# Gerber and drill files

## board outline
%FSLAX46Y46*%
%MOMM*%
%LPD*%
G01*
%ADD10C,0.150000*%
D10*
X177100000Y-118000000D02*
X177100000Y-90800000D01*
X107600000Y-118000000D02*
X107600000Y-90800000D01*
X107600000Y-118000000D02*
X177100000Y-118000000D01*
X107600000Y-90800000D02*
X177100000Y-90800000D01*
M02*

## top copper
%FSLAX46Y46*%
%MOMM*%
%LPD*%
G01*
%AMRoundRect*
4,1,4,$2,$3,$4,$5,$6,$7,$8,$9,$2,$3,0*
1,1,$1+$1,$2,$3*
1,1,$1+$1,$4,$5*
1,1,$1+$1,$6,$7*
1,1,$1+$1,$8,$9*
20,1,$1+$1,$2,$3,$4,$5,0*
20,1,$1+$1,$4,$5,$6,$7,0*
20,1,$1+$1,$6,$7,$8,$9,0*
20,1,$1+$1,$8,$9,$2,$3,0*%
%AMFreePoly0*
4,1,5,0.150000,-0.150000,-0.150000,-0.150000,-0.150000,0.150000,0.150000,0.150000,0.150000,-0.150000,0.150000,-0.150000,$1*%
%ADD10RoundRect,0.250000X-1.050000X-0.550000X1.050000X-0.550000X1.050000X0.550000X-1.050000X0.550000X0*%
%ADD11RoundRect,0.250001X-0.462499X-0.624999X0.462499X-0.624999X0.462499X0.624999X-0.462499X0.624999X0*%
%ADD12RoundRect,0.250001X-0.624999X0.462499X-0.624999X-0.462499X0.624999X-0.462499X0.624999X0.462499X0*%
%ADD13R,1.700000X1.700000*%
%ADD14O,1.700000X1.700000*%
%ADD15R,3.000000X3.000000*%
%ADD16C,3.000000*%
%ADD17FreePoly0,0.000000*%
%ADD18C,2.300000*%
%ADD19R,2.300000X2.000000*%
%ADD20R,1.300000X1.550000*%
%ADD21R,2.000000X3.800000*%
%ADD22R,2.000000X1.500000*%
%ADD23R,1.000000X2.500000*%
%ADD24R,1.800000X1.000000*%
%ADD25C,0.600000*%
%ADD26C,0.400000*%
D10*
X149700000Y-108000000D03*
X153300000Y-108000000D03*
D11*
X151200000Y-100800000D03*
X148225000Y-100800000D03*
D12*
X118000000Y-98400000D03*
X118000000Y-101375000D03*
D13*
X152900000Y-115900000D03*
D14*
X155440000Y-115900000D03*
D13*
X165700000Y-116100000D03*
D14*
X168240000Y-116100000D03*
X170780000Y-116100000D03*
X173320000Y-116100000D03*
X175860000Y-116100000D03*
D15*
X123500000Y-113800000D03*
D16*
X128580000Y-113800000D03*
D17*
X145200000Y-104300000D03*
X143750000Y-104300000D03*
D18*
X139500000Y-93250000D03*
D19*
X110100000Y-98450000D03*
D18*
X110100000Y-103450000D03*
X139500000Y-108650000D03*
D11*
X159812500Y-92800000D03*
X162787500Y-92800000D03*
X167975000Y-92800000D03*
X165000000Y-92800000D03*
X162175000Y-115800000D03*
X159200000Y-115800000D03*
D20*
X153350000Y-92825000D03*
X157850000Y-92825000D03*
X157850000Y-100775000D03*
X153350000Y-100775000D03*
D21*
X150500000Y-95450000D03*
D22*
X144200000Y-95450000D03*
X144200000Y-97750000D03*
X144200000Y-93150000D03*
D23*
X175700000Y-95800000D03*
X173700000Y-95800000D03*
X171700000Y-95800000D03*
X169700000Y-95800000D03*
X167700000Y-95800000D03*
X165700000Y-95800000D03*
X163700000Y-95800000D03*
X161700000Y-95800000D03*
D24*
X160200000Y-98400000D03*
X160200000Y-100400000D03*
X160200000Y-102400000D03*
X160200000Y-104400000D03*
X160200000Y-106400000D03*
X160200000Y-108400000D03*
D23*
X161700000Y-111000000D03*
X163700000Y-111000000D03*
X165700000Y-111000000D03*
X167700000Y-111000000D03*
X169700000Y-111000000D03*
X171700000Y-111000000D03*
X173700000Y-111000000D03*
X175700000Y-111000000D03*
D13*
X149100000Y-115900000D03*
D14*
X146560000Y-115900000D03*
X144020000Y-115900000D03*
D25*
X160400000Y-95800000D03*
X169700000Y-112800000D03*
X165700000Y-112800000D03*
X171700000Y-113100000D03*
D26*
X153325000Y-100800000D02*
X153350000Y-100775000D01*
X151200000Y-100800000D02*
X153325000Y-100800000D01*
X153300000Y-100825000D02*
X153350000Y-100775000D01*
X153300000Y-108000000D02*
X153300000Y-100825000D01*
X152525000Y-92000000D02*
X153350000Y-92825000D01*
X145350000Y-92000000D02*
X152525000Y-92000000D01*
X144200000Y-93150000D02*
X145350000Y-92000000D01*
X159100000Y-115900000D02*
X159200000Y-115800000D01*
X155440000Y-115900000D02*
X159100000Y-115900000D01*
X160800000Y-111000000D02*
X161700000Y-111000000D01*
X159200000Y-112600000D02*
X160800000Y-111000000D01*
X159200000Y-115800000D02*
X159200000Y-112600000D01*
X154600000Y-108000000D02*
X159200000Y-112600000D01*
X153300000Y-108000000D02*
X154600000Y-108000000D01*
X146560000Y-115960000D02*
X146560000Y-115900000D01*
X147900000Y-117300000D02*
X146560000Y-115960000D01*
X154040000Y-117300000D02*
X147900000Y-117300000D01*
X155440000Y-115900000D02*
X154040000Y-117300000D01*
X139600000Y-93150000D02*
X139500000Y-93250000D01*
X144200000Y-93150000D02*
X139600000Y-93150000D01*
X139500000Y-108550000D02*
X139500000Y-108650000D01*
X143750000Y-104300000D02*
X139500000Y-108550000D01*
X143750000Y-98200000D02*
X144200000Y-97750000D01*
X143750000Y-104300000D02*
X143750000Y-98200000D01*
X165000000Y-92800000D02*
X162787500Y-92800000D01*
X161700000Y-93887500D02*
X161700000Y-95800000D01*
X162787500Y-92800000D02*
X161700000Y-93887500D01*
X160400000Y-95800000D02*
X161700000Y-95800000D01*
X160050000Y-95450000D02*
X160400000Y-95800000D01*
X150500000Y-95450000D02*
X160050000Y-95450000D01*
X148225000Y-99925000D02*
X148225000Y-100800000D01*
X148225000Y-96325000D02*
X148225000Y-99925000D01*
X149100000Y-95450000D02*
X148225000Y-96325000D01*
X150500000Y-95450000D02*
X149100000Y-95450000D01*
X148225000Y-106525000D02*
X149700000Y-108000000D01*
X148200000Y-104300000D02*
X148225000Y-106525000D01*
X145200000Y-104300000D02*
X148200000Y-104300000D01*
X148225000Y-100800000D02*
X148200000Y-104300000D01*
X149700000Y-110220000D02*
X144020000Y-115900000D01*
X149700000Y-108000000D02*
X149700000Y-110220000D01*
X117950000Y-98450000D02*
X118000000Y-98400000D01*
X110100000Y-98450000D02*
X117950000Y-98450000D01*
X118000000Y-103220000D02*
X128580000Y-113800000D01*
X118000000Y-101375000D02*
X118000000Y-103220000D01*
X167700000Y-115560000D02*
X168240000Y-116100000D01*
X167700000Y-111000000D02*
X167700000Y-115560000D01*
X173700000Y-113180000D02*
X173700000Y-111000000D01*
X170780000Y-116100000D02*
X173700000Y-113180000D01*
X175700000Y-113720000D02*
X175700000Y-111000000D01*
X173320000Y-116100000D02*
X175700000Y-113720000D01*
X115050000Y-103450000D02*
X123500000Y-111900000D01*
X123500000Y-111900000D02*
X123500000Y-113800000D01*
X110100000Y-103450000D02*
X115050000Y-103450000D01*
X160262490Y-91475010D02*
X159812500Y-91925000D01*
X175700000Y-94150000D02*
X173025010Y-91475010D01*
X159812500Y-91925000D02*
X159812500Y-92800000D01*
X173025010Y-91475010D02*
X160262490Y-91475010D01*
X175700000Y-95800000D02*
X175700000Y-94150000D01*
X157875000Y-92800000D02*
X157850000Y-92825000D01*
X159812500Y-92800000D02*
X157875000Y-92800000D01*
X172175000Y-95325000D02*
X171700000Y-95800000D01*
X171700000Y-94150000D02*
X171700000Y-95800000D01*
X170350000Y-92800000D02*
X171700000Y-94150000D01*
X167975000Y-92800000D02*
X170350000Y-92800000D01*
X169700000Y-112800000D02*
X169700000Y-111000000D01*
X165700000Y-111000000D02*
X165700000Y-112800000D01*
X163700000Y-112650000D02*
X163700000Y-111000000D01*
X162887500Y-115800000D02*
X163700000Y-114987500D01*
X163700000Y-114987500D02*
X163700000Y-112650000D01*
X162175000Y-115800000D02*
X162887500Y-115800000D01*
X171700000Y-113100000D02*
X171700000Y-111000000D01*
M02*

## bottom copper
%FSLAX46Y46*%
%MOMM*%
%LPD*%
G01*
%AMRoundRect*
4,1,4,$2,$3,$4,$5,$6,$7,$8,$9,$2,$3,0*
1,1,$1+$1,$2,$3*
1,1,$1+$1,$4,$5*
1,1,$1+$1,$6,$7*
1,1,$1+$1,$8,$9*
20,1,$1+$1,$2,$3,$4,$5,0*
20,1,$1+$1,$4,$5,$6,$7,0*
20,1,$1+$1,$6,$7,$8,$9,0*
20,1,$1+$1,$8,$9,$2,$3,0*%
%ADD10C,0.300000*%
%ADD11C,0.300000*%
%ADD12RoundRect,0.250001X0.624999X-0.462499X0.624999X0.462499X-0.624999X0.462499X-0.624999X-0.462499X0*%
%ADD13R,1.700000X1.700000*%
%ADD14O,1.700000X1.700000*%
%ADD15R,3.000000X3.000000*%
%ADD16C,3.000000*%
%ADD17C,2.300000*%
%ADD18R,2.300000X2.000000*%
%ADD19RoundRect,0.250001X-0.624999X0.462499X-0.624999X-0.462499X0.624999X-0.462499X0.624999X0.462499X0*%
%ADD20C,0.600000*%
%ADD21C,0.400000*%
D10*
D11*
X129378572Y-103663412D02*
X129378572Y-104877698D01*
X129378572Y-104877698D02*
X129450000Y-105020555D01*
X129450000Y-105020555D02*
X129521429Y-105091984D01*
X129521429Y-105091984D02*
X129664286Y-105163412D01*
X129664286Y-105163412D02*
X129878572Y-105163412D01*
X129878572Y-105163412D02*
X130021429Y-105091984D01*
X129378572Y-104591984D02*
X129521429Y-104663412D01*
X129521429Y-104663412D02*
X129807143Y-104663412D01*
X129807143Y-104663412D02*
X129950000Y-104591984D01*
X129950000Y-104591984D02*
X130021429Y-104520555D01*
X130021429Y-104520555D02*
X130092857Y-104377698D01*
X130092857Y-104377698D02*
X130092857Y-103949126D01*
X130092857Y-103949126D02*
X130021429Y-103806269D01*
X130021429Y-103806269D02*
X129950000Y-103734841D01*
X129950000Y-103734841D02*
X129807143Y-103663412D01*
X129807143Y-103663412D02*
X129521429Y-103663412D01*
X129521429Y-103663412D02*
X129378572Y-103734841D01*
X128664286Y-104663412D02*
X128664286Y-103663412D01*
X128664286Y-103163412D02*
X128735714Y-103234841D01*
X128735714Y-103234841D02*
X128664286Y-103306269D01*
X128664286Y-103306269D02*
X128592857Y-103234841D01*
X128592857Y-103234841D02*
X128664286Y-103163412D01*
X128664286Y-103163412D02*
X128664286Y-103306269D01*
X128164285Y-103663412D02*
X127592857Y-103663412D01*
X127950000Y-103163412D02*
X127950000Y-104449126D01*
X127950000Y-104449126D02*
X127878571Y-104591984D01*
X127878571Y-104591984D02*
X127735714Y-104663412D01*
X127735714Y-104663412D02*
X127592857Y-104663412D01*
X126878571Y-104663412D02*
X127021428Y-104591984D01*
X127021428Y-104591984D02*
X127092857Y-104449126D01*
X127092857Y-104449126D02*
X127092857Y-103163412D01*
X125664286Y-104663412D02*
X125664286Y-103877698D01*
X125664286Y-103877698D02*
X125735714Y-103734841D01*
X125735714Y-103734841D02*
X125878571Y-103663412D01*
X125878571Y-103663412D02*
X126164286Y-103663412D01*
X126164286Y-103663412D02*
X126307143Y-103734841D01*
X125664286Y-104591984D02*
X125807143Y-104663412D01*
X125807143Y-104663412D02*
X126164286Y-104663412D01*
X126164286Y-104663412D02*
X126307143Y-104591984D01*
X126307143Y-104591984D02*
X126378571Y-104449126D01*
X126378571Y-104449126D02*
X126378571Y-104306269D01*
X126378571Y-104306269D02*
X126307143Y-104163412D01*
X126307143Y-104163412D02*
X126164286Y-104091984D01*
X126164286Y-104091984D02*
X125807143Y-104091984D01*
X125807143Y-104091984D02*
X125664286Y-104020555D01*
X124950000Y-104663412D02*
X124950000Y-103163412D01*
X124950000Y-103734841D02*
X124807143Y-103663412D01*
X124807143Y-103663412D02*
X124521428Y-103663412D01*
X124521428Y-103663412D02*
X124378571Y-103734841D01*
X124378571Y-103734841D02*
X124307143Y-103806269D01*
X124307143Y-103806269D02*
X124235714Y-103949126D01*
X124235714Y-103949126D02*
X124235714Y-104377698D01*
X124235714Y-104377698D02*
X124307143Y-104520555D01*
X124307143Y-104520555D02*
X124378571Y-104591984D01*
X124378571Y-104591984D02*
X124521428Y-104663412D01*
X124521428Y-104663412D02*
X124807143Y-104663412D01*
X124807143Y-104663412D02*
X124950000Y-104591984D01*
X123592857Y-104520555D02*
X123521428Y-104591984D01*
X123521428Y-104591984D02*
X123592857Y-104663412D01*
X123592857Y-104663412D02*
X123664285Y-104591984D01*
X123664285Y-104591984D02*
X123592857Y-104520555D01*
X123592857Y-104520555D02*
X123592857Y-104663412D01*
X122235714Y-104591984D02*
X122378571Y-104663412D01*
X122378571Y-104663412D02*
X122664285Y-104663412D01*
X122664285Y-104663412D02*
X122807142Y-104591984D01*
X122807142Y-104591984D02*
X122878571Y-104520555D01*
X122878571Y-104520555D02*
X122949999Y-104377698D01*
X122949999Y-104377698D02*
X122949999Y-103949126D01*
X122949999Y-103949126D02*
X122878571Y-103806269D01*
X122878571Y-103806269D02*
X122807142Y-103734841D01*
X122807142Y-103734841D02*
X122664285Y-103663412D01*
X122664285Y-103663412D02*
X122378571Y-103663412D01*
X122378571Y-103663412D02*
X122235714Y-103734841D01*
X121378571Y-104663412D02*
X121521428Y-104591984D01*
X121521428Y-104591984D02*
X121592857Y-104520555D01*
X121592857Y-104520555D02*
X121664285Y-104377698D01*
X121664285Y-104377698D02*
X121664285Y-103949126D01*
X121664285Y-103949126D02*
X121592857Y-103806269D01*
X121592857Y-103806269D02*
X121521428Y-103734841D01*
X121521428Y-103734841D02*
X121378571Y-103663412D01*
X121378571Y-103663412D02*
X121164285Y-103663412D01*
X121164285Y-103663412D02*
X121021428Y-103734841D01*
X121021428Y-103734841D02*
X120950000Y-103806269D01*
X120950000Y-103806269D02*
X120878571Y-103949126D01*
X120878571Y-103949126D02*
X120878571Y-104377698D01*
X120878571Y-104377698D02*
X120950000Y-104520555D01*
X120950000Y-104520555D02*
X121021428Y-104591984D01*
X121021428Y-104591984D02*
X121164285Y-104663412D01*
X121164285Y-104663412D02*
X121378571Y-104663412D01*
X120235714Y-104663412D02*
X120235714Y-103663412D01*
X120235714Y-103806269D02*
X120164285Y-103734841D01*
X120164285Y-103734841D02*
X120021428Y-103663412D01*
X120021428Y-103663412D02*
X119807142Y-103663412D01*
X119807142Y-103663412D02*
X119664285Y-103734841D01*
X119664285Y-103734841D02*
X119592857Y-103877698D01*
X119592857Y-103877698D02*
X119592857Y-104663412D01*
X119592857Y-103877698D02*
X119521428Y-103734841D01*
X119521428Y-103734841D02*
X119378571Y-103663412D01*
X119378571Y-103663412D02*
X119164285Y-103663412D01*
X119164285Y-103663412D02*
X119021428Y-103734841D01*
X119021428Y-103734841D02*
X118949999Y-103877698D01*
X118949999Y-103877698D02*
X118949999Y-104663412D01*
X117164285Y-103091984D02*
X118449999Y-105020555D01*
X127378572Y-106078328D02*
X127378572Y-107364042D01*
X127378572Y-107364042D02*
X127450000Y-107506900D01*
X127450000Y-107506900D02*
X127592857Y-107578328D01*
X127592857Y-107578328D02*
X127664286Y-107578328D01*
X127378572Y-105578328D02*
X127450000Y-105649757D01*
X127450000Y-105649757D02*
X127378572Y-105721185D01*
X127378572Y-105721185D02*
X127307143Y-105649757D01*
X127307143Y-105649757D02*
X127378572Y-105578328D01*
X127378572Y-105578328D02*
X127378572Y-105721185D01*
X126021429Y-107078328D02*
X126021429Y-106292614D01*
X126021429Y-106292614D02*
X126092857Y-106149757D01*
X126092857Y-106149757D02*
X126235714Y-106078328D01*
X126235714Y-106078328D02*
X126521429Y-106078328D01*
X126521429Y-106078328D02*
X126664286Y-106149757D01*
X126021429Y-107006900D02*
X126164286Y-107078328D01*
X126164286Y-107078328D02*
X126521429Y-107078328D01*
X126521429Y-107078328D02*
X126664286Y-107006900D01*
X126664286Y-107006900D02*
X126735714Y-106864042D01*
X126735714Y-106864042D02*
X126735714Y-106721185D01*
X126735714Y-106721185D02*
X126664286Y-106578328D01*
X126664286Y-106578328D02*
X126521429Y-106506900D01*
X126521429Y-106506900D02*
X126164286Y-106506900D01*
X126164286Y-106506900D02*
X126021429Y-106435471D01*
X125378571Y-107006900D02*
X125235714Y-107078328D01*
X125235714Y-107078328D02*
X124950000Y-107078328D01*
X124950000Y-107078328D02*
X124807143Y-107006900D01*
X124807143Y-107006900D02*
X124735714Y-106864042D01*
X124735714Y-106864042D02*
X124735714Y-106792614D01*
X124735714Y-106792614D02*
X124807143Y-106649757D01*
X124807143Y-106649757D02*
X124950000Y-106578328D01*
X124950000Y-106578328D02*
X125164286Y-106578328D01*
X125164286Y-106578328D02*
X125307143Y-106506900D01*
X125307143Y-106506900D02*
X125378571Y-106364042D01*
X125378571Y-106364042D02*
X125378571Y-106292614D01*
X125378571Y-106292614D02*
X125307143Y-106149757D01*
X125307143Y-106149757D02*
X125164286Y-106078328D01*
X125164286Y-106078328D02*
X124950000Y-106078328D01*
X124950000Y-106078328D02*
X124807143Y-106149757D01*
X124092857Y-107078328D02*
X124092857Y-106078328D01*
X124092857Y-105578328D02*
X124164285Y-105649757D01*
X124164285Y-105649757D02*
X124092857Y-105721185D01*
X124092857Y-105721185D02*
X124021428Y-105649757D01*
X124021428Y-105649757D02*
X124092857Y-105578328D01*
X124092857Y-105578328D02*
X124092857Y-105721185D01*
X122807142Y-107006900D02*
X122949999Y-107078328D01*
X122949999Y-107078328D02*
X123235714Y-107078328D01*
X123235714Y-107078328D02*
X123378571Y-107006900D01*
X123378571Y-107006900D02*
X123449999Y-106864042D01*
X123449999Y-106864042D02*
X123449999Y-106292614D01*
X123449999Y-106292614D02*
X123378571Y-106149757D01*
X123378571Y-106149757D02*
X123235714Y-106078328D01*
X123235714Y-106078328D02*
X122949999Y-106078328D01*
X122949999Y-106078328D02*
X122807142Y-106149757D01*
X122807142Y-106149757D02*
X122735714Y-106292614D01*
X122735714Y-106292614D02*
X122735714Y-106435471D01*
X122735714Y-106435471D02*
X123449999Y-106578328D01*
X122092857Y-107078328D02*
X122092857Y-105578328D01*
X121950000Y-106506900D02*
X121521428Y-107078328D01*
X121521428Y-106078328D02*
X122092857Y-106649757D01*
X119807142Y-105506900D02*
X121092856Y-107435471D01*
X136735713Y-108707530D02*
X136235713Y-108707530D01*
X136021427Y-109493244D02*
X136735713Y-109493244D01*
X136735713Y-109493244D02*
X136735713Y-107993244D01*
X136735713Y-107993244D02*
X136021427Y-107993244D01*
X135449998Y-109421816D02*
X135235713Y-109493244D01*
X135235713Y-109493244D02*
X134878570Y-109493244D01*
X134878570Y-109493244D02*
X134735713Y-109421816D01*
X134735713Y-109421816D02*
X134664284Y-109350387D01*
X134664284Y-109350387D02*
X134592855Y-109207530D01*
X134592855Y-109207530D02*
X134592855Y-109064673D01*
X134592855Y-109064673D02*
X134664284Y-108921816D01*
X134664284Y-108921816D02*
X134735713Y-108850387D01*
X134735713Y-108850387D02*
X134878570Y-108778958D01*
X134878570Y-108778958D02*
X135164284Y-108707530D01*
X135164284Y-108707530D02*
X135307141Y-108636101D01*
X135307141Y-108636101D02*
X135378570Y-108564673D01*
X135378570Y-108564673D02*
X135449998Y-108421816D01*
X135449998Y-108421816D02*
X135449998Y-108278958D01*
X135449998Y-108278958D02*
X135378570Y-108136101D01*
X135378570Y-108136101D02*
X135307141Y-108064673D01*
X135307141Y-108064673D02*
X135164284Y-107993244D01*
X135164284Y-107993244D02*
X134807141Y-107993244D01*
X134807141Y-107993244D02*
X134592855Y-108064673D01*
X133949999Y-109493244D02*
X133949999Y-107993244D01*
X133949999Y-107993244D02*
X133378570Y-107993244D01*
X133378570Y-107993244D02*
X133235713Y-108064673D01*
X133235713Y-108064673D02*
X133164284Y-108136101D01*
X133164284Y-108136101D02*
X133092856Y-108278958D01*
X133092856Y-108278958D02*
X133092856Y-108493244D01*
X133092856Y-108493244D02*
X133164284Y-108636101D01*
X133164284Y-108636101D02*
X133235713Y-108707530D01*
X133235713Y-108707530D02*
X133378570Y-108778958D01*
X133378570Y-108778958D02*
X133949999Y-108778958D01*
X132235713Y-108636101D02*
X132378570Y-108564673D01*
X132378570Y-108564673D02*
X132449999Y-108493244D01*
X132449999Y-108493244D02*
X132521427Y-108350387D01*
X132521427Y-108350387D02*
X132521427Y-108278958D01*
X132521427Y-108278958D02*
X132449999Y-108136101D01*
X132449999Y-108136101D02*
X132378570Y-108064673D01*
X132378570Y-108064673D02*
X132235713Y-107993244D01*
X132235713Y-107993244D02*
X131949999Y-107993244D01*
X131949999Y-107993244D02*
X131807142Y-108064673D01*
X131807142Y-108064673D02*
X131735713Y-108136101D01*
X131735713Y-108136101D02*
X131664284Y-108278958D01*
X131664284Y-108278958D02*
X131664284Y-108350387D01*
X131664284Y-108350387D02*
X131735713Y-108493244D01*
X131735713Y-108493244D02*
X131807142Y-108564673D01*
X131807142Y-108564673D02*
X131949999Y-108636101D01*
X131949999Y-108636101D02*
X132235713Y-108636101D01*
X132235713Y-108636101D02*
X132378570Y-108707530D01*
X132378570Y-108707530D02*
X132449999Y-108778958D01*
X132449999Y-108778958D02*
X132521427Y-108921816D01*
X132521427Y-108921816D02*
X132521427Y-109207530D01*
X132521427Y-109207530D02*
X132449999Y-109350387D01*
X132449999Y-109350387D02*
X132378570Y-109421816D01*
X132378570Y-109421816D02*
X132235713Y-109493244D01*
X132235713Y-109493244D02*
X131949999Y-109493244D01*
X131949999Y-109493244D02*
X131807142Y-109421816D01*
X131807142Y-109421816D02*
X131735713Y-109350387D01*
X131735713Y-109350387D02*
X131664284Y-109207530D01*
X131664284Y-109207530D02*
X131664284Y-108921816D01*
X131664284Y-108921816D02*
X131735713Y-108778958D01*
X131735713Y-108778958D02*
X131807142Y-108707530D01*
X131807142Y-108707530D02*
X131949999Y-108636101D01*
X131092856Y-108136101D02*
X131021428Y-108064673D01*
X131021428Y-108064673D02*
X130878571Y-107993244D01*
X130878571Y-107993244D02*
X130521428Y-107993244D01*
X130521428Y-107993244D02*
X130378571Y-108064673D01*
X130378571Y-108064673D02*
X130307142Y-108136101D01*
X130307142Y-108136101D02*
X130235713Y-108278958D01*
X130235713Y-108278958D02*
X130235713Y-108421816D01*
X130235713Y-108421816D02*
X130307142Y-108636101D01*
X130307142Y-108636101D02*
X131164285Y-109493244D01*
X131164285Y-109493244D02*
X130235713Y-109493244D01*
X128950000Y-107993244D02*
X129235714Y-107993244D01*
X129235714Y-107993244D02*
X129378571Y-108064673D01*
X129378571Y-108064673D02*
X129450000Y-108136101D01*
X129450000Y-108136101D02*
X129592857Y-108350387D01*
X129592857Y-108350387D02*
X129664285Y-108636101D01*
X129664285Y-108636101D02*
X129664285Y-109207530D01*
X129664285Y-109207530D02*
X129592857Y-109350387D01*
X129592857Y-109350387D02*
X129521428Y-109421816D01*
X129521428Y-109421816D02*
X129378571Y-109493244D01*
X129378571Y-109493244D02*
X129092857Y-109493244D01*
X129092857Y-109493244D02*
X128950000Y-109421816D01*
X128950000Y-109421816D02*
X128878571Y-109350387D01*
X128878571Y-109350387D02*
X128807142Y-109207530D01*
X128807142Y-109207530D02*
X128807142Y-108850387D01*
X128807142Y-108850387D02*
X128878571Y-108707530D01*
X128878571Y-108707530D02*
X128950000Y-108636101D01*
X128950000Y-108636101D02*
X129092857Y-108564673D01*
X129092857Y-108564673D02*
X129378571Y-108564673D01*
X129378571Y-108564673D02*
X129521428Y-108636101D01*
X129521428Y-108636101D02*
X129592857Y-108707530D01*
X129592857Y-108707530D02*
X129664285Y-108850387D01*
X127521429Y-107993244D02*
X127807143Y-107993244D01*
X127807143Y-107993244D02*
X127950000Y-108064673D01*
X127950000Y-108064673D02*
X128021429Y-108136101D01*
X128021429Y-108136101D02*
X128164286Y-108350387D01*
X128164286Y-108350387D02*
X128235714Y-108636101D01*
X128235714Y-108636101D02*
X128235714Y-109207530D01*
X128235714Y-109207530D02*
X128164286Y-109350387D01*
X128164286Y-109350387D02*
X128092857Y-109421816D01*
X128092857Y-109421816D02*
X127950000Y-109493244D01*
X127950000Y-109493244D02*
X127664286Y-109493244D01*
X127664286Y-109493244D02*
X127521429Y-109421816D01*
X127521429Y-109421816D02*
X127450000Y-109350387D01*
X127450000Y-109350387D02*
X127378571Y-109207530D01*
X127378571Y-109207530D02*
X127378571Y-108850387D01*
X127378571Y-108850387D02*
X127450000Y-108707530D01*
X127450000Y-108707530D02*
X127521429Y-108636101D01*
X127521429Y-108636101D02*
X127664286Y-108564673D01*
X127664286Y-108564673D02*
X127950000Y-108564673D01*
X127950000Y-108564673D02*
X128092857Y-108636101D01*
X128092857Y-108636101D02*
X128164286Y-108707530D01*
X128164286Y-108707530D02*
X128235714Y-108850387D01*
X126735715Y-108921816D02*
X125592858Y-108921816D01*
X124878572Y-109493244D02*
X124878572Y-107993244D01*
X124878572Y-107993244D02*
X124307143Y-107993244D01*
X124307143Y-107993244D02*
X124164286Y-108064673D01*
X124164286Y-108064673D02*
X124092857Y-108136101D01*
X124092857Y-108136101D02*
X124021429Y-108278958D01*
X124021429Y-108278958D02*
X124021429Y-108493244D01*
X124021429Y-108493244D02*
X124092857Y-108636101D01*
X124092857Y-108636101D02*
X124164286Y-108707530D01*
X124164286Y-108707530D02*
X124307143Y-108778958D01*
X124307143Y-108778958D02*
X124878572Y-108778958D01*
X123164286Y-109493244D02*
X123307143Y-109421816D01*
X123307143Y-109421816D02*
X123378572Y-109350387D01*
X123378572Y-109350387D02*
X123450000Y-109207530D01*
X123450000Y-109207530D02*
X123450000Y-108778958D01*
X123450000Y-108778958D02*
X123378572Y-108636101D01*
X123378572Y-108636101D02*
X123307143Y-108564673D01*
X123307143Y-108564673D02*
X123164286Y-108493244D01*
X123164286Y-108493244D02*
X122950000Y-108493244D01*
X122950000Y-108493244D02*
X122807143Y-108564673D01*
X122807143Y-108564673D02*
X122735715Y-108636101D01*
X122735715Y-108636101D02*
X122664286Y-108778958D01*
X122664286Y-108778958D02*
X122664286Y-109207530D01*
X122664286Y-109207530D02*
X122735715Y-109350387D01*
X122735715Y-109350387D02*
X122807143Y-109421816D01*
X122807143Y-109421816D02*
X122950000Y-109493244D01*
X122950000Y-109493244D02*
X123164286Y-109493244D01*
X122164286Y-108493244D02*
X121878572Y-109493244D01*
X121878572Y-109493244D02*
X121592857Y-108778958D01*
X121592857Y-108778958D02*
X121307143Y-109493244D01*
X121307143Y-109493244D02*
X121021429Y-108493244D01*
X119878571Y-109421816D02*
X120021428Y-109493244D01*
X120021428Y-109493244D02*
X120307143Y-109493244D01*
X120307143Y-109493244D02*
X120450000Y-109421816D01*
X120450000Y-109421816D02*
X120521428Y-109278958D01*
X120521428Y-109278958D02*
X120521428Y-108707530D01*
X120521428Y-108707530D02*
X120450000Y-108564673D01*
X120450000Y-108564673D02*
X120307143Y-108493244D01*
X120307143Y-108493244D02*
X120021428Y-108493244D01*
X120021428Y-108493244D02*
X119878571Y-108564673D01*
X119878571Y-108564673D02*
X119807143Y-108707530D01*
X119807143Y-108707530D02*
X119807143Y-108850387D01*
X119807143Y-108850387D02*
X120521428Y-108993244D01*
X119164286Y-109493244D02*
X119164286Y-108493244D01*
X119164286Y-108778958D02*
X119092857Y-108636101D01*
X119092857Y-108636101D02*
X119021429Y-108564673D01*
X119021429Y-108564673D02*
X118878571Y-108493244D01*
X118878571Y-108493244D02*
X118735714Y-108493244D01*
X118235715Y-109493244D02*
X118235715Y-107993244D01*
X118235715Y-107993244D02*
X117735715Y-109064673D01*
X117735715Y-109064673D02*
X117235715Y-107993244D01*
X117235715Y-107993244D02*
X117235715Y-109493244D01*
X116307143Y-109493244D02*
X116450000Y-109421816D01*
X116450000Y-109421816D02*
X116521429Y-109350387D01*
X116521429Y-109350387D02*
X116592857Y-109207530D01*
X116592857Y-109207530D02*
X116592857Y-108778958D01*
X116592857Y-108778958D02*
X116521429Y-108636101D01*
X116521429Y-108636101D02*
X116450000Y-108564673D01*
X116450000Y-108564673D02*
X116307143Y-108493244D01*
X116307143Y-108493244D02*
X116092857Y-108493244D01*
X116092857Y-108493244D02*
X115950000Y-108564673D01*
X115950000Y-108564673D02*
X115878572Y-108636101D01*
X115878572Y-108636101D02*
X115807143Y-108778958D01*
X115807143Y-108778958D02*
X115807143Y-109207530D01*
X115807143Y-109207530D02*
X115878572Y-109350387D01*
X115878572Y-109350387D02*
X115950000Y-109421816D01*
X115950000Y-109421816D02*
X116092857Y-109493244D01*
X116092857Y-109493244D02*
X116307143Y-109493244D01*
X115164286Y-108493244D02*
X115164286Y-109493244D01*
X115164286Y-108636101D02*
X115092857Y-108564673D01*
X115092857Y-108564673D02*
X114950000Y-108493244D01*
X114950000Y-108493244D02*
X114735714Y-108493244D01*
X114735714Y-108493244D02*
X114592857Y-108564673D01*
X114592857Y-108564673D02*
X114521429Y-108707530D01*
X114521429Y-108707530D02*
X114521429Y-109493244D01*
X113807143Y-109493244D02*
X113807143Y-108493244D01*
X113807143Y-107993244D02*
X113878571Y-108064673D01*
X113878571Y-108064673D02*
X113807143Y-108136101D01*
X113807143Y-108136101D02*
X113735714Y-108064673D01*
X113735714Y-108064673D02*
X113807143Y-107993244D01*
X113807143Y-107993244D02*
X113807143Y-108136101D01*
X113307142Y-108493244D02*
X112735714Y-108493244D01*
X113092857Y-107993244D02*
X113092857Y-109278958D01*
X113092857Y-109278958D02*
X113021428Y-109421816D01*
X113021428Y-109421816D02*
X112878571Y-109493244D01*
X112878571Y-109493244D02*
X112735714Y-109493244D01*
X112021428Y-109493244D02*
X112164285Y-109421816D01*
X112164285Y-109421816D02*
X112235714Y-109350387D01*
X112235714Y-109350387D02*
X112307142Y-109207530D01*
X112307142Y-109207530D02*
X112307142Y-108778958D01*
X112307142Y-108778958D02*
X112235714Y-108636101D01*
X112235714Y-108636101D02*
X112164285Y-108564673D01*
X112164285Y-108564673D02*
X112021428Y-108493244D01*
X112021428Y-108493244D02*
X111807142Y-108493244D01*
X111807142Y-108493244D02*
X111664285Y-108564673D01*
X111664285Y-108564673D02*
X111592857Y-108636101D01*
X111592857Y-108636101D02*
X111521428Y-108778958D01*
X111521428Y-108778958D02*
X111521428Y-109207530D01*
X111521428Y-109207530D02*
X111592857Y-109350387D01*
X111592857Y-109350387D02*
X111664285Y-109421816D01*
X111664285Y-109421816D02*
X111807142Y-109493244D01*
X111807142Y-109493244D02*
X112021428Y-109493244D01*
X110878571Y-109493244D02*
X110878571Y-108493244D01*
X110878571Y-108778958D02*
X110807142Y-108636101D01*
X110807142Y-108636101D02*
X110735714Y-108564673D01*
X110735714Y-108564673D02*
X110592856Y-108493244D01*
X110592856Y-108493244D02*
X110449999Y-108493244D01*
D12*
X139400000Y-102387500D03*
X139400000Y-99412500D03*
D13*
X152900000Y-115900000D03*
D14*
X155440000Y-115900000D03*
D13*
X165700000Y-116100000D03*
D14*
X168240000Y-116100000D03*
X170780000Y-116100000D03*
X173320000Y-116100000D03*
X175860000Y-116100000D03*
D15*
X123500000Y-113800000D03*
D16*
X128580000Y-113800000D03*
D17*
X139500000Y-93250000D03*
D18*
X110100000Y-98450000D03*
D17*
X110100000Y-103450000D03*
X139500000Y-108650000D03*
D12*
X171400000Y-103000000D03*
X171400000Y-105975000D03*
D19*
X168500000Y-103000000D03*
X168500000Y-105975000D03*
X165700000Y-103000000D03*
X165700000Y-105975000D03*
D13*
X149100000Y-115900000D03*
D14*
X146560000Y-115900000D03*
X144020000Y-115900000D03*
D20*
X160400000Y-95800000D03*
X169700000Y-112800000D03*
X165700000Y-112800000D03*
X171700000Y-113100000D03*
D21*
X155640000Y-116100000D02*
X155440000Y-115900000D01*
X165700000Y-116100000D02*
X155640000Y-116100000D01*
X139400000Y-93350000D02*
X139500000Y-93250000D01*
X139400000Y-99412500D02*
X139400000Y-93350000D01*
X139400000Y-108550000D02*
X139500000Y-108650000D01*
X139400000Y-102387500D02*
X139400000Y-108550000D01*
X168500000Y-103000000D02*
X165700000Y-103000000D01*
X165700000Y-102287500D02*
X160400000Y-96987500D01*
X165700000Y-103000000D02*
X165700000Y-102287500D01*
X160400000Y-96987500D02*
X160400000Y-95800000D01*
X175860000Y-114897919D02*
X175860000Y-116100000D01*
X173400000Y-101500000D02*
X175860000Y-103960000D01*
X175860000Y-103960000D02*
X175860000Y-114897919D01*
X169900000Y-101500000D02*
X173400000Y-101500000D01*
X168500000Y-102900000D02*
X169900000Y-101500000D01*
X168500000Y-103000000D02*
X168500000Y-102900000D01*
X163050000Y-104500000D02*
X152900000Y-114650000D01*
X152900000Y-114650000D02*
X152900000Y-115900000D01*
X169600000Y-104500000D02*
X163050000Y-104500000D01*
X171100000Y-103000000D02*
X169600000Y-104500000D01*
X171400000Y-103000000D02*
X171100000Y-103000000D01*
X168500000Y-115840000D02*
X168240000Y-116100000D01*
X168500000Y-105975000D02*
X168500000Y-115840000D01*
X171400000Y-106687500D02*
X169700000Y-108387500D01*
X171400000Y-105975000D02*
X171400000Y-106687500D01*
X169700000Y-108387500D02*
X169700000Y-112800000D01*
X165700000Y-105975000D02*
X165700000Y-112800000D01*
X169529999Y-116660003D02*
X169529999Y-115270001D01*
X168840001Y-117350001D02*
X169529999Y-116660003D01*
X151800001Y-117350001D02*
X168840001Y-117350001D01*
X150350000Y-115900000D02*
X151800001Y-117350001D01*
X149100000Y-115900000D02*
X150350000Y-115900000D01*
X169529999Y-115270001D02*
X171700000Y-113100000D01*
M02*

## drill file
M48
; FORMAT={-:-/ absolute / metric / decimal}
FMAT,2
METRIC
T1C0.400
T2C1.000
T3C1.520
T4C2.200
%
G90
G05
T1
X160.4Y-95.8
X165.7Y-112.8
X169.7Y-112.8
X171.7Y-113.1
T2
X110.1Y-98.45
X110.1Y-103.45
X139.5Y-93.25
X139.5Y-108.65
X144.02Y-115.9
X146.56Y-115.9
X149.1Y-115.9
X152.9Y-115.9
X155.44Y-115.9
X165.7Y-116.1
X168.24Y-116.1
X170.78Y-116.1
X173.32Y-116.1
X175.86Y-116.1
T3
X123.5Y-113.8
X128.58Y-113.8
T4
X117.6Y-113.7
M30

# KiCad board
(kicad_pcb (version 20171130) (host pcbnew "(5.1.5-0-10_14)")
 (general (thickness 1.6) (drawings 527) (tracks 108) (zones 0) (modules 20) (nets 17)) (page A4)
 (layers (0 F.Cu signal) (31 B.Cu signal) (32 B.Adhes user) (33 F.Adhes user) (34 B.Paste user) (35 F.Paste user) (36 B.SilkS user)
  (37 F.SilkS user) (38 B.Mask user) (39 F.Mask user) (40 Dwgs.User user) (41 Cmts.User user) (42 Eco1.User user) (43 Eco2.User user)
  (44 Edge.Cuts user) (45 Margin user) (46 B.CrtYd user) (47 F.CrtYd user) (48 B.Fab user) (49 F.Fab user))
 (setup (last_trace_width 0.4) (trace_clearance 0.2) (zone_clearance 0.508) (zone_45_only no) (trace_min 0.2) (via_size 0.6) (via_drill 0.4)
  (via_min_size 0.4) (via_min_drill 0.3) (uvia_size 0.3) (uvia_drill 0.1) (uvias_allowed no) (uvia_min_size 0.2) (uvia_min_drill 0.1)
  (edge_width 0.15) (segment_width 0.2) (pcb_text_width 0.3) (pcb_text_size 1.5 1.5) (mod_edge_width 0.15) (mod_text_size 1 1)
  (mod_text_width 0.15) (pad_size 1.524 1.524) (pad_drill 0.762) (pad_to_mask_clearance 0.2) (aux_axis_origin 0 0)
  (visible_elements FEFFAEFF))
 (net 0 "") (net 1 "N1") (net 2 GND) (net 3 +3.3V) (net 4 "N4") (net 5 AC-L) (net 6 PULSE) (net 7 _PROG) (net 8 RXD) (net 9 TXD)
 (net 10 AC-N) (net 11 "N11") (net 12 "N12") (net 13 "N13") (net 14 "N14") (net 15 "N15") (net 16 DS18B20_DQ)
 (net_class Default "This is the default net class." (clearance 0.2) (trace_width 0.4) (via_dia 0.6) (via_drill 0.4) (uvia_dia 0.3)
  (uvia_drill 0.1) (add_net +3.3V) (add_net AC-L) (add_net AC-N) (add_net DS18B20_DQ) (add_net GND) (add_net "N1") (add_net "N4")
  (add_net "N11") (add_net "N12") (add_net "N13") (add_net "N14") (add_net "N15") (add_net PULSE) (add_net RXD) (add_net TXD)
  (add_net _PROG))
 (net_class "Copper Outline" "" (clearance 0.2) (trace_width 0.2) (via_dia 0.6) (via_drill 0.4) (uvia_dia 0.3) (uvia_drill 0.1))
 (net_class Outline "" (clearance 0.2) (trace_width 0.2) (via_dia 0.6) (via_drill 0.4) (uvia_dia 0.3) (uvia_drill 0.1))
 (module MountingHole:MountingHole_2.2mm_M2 (layer F.Cu) (at 117.6 113.7)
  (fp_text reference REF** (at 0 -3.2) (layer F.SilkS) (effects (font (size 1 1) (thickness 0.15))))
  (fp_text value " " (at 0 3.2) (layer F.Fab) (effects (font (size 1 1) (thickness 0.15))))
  (pad 1 np_thru_hole circle (at 0 0) (size 2.2 2.2) (drill 2.2) (layers *.Cu *.Mask)))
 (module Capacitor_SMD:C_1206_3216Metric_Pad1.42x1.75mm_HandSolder (layer B.Cu) (at 139.4 100.9 90)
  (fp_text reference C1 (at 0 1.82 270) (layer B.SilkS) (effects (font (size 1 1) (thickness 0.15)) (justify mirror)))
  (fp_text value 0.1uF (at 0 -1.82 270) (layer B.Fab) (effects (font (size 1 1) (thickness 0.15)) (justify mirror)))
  (pad 1 smd roundrect (at -1.4875 0 90) (size 1.425 1.75) (layers B.Cu B.Paste B.Mask) (roundrect_rratio 0.175439) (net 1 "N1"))
  (pad 2 smd roundrect (at 1.4875 0 90) (size 1.425 1.75) (layers B.Cu B.Paste B.Mask) (roundrect_rratio 0.175439) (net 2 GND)))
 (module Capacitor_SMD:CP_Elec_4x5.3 (layer F.Cu) (at 151.5 108)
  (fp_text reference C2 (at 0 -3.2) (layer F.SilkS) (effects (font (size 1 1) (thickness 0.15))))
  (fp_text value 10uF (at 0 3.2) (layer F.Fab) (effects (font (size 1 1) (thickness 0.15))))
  (pad 1 smd roundrect (at -1.8 0) (size 2.6 1.6) (layers F.Cu F.Paste F.Mask) (roundrect_rratio 0.15625) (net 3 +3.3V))
  (pad 2 smd roundrect (at 1.8 0) (size 2.6 1.6) (layers F.Cu F.Paste F.Mask) (roundrect_rratio 0.15625) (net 2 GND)))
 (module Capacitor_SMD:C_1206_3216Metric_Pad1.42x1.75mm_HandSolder (layer F.Cu) (at 149.7125 100.8)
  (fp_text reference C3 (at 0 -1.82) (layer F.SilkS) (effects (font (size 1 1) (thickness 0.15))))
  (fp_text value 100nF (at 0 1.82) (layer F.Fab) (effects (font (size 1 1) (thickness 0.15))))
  (pad 2 smd roundrect (at 1.4875 0) (size 1.425 1.75) (layers F.Cu F.Paste F.Mask) (roundrect_rratio 0.175439) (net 2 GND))
  (pad 1 smd roundrect (at -1.4875 0) (size 1.425 1.75) (layers F.Cu F.Paste F.Mask) (roundrect_rratio 0.175439) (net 3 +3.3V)))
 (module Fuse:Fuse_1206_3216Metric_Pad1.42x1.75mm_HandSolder (layer F.Cu) (at 118 99.8875 270)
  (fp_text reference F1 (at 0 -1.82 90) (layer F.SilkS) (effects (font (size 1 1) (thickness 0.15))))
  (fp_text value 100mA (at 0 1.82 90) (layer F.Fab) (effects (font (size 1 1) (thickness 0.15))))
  (pad 1 smd roundrect (at -1.4875 0 270) (size 1.425 1.75) (layers F.Cu F.Paste F.Mask) (roundrect_rratio 0.175439) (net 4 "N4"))
  (pad 2 smd roundrect (at 1.4875 0 270) (size 1.425 1.75) (layers F.Cu F.Paste F.Mask) (roundrect_rratio 0.175439) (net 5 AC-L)))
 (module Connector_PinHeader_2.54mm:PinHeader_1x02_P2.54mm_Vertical (layer F.Cu) (at 152.9 115.9 90)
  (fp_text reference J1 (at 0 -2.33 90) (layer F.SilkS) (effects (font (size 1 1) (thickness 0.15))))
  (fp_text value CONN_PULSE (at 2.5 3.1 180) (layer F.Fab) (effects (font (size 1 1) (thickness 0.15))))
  (pad 1 thru_hole rect (at 0 0 90) (size 1.7 1.7) (drill 1) (layers *.Cu *.Mask) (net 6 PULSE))
  (pad 2 thru_hole oval (at 0 2.54 90) (size 1.7 1.7) (drill 1) (layers *.Cu *.Mask) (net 2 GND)))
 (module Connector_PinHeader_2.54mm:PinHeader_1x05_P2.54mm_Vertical (layer F.Cu) (at 165.7 116.1 90)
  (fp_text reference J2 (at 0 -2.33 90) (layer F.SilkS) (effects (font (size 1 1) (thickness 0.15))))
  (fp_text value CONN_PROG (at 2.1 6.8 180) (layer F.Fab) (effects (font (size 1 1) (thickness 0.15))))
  (pad 1 thru_hole rect (at 0 0 90) (size 1.7 1.7) (drill 1) (layers *.Cu *.Mask) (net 2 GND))
  (pad 2 thru_hole oval (at 0 2.54 90) (size 1.7 1.7) (drill 1) (layers *.Cu *.Mask) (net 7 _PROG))
  (pad 3 thru_hole oval (at 0 5.08 90) (size 1.7 1.7) (drill 1) (layers *.Cu *.Mask) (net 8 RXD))
  (pad 4 thru_hole oval (at 0 7.62 90) (size 1.7 1.7) (drill 1) (layers *.Cu *.Mask) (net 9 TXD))
  (pad 5 thru_hole oval (at 0 10.16 90) (size 1.7 1.7) (drill 1) (layers *.Cu *.Mask) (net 3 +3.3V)))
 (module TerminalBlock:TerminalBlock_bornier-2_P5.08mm (layer F.Cu) (at 123.5 113.8)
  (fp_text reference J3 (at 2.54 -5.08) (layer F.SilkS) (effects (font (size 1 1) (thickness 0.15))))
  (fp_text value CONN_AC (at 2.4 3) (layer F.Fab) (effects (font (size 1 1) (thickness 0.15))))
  (pad 1 thru_hole rect (at 0 0) (size 3 3) (drill 1.52) (layers *.Cu *.Mask) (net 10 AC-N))
  (pad 2 thru_hole circle (at 5.08 0) (size 3 3) (drill 1.52) (layers *.Cu *.Mask) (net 5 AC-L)))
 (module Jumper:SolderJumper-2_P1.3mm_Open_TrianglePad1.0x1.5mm (layer F.Cu) (at 144.475 104.3)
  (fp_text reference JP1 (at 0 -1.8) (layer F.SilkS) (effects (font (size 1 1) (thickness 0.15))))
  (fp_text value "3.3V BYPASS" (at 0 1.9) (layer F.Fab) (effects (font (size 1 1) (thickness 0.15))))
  (pad 2 smd custom (at 0.725 0) (size 0.3 0.3) (layers F.Cu F.Mask) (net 3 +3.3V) (zone_connect 2)
   (options (clearance outline) (anchor rect)) (primitives))
  (pad 1 smd custom (at -0.725 0) (size 0.3 0.3) (layers F.Cu F.Mask) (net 1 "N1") (zone_connect 2)
   (options (clearance outline) (anchor rect)) (primitives)))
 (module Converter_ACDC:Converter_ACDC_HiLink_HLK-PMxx (layer F.Cu) (at 110.1 98.45)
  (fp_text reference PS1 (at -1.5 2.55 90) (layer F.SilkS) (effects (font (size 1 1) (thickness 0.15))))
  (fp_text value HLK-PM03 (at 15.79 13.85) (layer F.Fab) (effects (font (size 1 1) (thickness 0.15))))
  (pad 3 thru_hole circle (at 29.4 -5.2) (size 2.3 2.3) (drill 1) (layers *.Cu *.Mask) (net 2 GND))
  (pad 1 thru_hole rect (at 0 0) (size 2.3 2) (drill 1) (layers *.Cu *.Mask) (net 4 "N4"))
  (pad 2 thru_hole circle (at 0 5) (size 2.3 2.3) (drill 1) (layers *.Cu *.Mask) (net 10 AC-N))
  (pad 4 thru_hole circle (at 29.4 10.2) (size 2.3 2.3) (drill 1) (layers *.Cu *.Mask) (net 1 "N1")))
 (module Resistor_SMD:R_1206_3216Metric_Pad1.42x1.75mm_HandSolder (layer F.Cu) (at 161.3 92.8)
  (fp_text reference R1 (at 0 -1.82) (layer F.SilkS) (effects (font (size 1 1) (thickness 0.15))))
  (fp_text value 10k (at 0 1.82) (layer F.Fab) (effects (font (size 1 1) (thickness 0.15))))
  (pad 1 smd roundrect (at -1.4875 0) (size 1.425 1.75) (layers F.Cu F.Paste F.Mask) (roundrect_rratio 0.175439) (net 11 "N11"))
  (pad 2 smd roundrect (at 1.4875 0) (size 1.425 1.75) (layers F.Cu F.Paste F.Mask) (roundrect_rratio 0.175439) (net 3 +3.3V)))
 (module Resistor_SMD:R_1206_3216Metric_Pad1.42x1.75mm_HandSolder (layer F.Cu) (at 166.4875 92.8)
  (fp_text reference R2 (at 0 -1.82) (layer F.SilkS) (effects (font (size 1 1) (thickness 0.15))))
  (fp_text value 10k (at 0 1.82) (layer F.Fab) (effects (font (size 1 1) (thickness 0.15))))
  (pad 2 smd roundrect (at 1.4875 0) (size 1.425 1.75) (layers F.Cu F.Paste F.Mask) (roundrect_rratio 0.175439) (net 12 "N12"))
  (pad 1 smd roundrect (at -1.4875 0) (size 1.425 1.75) (layers F.Cu F.Paste F.Mask) (roundrect_rratio 0.175439) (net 3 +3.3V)))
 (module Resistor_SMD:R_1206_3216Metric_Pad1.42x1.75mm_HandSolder (layer B.Cu) (at 171.4 104.4875 90)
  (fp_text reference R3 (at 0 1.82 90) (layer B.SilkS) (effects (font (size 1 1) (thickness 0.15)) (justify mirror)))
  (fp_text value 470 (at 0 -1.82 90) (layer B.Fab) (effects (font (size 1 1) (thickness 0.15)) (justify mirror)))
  (pad 2 smd roundrect (at 1.4875 0 90) (size 1.425 1.75) (layers B.Cu B.Paste B.Mask) (roundrect_rratio 0.175439) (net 6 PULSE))
  (pad 1 smd roundrect (at -1.4875 0 90) (size 1.425 1.75) (layers B.Cu B.Paste B.Mask) (roundrect_rratio 0.175439) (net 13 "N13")))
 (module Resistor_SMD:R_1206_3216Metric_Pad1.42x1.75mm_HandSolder (layer B.Cu) (at 168.5 104.4875 270)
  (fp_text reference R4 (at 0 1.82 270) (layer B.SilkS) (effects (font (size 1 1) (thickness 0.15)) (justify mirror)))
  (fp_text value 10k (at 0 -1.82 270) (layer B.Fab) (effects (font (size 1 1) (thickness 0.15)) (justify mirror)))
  (pad 1 smd roundrect (at -1.4875 0 270) (size 1.425 1.75) (layers B.Cu B.Paste B.Mask) (roundrect_rratio 0.175439) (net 3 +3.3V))
  (pad 2 smd roundrect (at 1.4875 0 270) (size 1.425 1.75) (layers B.Cu B.Paste B.Mask) (roundrect_rratio 0.175439) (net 7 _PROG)))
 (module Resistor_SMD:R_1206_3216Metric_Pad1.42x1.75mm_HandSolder (layer B.Cu) (at 165.7 104.4875 270)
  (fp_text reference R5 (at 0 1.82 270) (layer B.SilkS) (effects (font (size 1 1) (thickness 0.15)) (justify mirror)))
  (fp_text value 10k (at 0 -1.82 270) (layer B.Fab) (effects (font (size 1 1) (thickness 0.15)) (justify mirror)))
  (pad 1 smd roundrect (at -1.4875 0 270) (size 1.425 1.75) (layers B.Cu B.Paste B.Mask) (roundrect_rratio 0.175439) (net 3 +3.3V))
  (pad 2 smd roundrect (at 1.4875 0 270) (size 1.425 1.75) (layers B.Cu B.Paste B.Mask) (roundrect_rratio 0.175439) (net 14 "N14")))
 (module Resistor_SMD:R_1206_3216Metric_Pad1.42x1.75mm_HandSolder (layer F.Cu) (at 160.6875 115.8)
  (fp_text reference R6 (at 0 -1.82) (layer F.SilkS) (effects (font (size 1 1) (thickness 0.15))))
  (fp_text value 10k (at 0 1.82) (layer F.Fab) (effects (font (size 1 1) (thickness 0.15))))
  (pad 2 smd roundrect (at 1.4875 0) (size 1.425 1.75) (layers F.Cu F.Paste F.Mask) (roundrect_rratio 0.175439) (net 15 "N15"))
  (pad 1 smd roundrect (at -1.4875 0) (size 1.425 1.75) (layers F.Cu F.Paste F.Mask) (roundrect_rratio 0.175439) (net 2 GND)))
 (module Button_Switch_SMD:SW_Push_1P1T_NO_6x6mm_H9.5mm (layer F.Cu) (at 155.6 96.8 270)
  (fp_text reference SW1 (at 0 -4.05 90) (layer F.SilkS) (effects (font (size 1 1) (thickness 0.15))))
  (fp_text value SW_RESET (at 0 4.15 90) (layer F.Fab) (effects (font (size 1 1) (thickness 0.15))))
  (pad 2 smd rect (at -3.975 2.25 270) (size 1.55 1.3) (layers F.Cu F.Paste F.Mask) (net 2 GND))
  (pad 1 smd rect (at -3.975 -2.25 270) (size 1.55 1.3) (layers F.Cu F.Paste F.Mask) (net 11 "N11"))
  (pad 1 smd rect (at 3.975 -2.25 270) (size 1.55 1.3) (layers F.Cu F.Paste F.Mask) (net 11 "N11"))
  (pad 2 smd rect (at 3.975 2.25 270) (size 1.55 1.3) (layers F.Cu F.Paste F.Mask) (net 2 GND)))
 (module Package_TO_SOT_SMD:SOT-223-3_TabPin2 (layer F.Cu) (at 147.35 95.45)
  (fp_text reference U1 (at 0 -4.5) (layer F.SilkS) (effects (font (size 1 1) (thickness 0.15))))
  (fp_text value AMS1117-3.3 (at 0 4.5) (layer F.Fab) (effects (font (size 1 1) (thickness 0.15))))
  (pad 2 smd rect (at 3.15 0) (size 2 3.8) (layers F.Cu F.Paste F.Mask) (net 3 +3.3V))
  (pad 2 smd rect (at -3.15 0) (size 2 1.5) (layers F.Cu F.Paste F.Mask) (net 3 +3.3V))
  (pad 3 smd rect (at -3.15 2.3) (size 2 1.5) (layers F.Cu F.Paste F.Mask) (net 1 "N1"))
  (pad 1 smd rect (at -3.15 -2.3) (size 2 1.5) (layers F.Cu F.Paste F.Mask) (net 2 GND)))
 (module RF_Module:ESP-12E (layer F.Cu) (at 172.2 103.4 270)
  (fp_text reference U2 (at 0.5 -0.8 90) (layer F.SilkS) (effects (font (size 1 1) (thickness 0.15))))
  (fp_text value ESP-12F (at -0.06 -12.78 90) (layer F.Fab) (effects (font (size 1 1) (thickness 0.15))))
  (pad 1 smd rect (at -7.6 -3.5 270) (size 2.5 1) (layers F.Cu F.Paste F.Mask) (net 11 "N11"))
  (pad 2 smd rect (at -7.6 -1.5 270) (size 2.5 1) (layers F.Cu F.Paste F.Mask))
  (pad 3 smd rect (at -7.6 0.5 270) (size 2.5 1) (layers F.Cu F.Paste F.Mask) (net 12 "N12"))
  (pad 4 smd rect (at -7.6 2.5 270) (size 2.5 1) (layers F.Cu F.Paste F.Mask))
  (pad 5 smd rect (at -7.6 4.5 270) (size 2.5 1) (layers F.Cu F.Paste F.Mask))
  (pad 6 smd rect (at -7.6 6.5 270) (size 2.5 1) (layers F.Cu F.Paste F.Mask))
  (pad 7 smd rect (at -7.6 8.5 270) (size 2.5 1) (layers F.Cu F.Paste F.Mask))
  (pad 8 smd rect (at -7.6 10.5 270) (size 2.5 1) (layers F.Cu F.Paste F.Mask) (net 3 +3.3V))
  (pad 9 smd rect (at -5 12 270) (size 1 1.8) (layers F.Cu F.Paste F.Mask))
  (pad 10 smd rect (at -3 12 270) (size 1 1.8) (layers F.Cu F.Paste F.Mask))
  (pad 11 smd rect (at -1 12 270) (size 1 1.8) (layers F.Cu F.Paste F.Mask))
  (pad 12 smd rect (at 1 12 270) (size 1 1.8) (layers F.Cu F.Paste F.Mask))
  (pad 13 smd rect (at 3 12 270) (size 1 1.8) (layers F.Cu F.Paste F.Mask))
  (pad 14 smd rect (at 5 12 270) (size 1 1.8) (layers F.Cu F.Paste F.Mask))
  (pad 15 smd rect (at 7.6 10.5 270) (size 2.5 1) (layers F.Cu F.Paste F.Mask) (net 2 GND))
  (pad 16 smd rect (at 7.6 8.5 270) (size 2.5 1) (layers F.Cu F.Paste F.Mask) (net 15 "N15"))
  (pad 17 smd rect (at 7.6 6.5 270) (size 2.5 1) (layers F.Cu F.Paste F.Mask) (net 14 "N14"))
  (pad 18 smd rect (at 7.6 4.5 270) (size 2.5 1) (layers F.Cu F.Paste F.Mask) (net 7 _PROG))
  (pad 19 smd rect (at 7.6 2.5 270) (size 2.5 1) (layers F.Cu F.Paste F.Mask) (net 13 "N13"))
  (pad 20 smd rect (at 7.6 0.5 270) (size 2.5 1) (layers F.Cu F.Paste F.Mask) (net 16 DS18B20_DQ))
  (pad 21 smd rect (at 7.6 -1.5 270) (size 2.5 1) (layers F.Cu F.Paste F.Mask) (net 8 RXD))
  (pad 22 smd rect (at 7.6 -3.5 270) (size 2.5 1) (layers F.Cu F.Paste F.Mask) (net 9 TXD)))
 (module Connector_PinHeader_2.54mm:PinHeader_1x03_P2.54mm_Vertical (layer F.Cu) (at 149.1 115.9 270)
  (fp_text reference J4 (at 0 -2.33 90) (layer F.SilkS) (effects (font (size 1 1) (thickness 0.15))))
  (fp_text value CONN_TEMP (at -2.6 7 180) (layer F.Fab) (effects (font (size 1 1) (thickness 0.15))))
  (pad 1 thru_hole rect (at 0 0 270) (size 1.7 1.7) (drill 1) (layers *.Cu *.Mask) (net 16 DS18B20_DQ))
  (pad 2 thru_hole oval (at 0 2.54 270) (size 1.7 1.7) (drill 1) (layers *.Cu *.Mask) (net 2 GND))
  (pad 3 thru_hole oval (at 0 5.08 270) (size 1.7 1.7) (drill 1) (layers *.Cu *.Mask) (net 3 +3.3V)))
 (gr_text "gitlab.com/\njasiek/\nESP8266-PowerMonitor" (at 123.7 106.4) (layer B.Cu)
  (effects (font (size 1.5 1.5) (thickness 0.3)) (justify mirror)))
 (gr_line (start 177.1 118) (end 177.1 90.8) (layer Edge.Cuts) (width 0.15))
 (gr_line (start 107.6 118) (end 107.6 90.8) (layer Edge.Cuts) (width 0.15))
 (gr_line (start 107.6 118) (end 177.1 118) (layer Edge.Cuts) (width 0.15))
 (gr_line (start 107.6 90.8) (end 177.1 90.8) (layer Edge.Cuts) (width 0.15))
 (segment (start 153.325 100.8) (end 153.35 100.775) (width 0.4) (layer F.Cu) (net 2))
 (segment (start 151.2 100.8) (end 153.325 100.8) (width 0.4) (layer F.Cu) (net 2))
 (segment (start 153.3 100.825) (end 153.35 100.775) (width 0.4) (layer F.Cu) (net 2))
 (segment (start 153.3 108) (end 153.3 100.825) (width 0.4) (layer F.Cu) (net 2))
 (segment (start 152.525 92) (end 153.35 92.825) (width 0.4) (layer F.Cu) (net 2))
 (segment (start 145.35 92) (end 152.525 92) (width 0.4) (layer F.Cu) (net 2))
 (segment (start 144.2 93.15) (end 145.35 92) (width 0.4) (layer F.Cu) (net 2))
 (segment (start 155.64 116.1) (end 155.44 115.9) (width 0.4) (layer B.Cu) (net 2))
 (segment (start 165.7 116.1) (end 155.64 116.1) (width 0.4) (layer B.Cu) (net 2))
 (segment (start 159.1 115.9) (end 159.2 115.8) (width 0.4) (layer F.Cu) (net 2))
 (segment (start 155.44 115.9) (end 159.1 115.9) (width 0.4) (layer F.Cu) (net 2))
 (segment (start 160.8 111) (end 161.7 111) (width 0.4) (layer F.Cu) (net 2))
 (segment (start 159.2 112.6) (end 160.8 111) (width 0.4) (layer F.Cu) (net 2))
 (segment (start 159.2 115.8) (end 159.2 112.6) (width 0.4) (layer F.Cu) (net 2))
 (segment (start 154.6 108) (end 159.2 112.6) (width 0.4) (layer F.Cu) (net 2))
 (segment (start 153.3 108) (end 154.6 108) (width 0.4) (layer F.Cu) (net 2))
 (segment (start 146.56 115.96) (end 146.56 115.9) (width 0.4) (layer F.Cu) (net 2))
 (segment (start 147.9 117.3) (end 146.56 115.96) (width 0.4) (layer F.Cu) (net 2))
 (segment (start 154.04 117.3) (end 147.9 117.3) (width 0.4) (layer F.Cu) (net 2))
 (segment (start 155.44 115.9) (end 154.04 117.3) (width 0.4) (layer F.Cu) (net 2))
 (segment (start 139.4 93.35) (end 139.5 93.25) (width 0.4) (layer B.Cu) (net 2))
 (segment (start 139.4 99.4125) (end 139.4 93.35) (width 0.4) (layer B.Cu) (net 2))
 (segment (start 139.6 93.15) (end 139.5 93.25) (width 0.4) (layer F.Cu) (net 2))
 (segment (start 144.2 93.15) (end 139.6 93.15) (width 0.4) (layer F.Cu) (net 2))
 (segment (start 139.4 108.55) (end 139.5 108.65) (width 0.4) (layer B.Cu) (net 1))
 (segment (start 139.4 102.3875) (end 139.4 108.55) (width 0.4) (layer B.Cu) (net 1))
 (segment (start 139.5 108.55) (end 139.5 108.65) (width 0.4) (layer F.Cu) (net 1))
 (segment (start 143.75 104.3) (end 139.5 108.55) (width 0.4) (layer F.Cu) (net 1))
 (segment (start 143.75 98.2) (end 144.2 97.75) (width 0.4) (layer F.Cu) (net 1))
 (segment (start 143.75 104.3) (end 143.75 98.2) (width 0.4) (layer F.Cu) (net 1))
 (segment (start 165 92.8) (end 162.7875 92.8) (width 0.4) (layer F.Cu) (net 3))
 (segment (start 161.7 93.8875) (end 161.7 95.8) (width 0.4) (layer F.Cu) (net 3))
 (segment (start 162.7875 92.8) (end 161.7 93.8875) (width 0.4) (layer F.Cu) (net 3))
 (segment (start 168.5 103) (end 165.7 103) (width 0.4) (layer B.Cu) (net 3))
 (segment (start 165.7 102.2875) (end 160.4 96.9875) (width 0.4) (layer B.Cu) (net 3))
 (segment (start 165.7 103) (end 165.7 102.2875) (width 0.4) (layer B.Cu) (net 3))
 (via (at 160.4 95.8) (size 0.6) (drill 0.4) (layers F.Cu B.Cu) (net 3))
 (segment (start 160.4 96.9875) (end 160.4 95.8) (width 0.4) (layer B.Cu) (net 3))
 (segment (start 160.4 95.8) (end 161.7 95.8) (width 0.4) (layer F.Cu) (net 3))
 (segment (start 160.05 95.45) (end 160.4 95.8) (width 0.4) (layer F.Cu) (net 3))
 (segment (start 150.5 95.45) (end 160.05 95.45) (width 0.4) (layer F.Cu) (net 3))
 (segment (start 148.225 99.925) (end 148.225 100.8) (width 0.4) (layer F.Cu) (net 3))
 (segment (start 148.225 96.325) (end 148.225 99.925) (width 0.4) (layer F.Cu) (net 3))
 (segment (start 149.1 95.45) (end 148.225 96.325) (width 0.4) (layer F.Cu) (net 3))
 (segment (start 150.5 95.45) (end 149.1 95.45) (width 0.4) (layer F.Cu) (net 3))
 (segment (start 148.225 106.525) (end 149.7 108) (width 0.4) (layer F.Cu) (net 3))
 (segment (start 148.2 104.3) (end 148.225 106.525) (width 0.4) (layer F.Cu) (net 3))
 (segment (start 145.2 104.3) (end 148.2 104.3) (width 0.4) (layer F.Cu) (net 3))
 (segment (start 148.225 100.8) (end 148.2 104.3) (width 0.4) (layer F.Cu) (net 3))
 (segment (start 175.86 114.897919) (end 175.86 116.1) (width 0.4) (layer B.Cu) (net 3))
 (segment (start 173.4 101.5) (end 175.86 103.96) (width 0.4) (layer B.Cu) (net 3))
 (segment (start 175.86 103.96) (end 175.86 114.897919) (width 0.4) (layer B.Cu) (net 3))
 (segment (start 169.9 101.5) (end 173.4 101.5) (width 0.4) (layer B.Cu) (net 3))
 (segment (start 168.5 102.9) (end 169.9 101.5) (width 0.4) (layer B.Cu) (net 3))
 (segment (start 168.5 103) (end 168.5 102.9) (width 0.4) (layer B.Cu) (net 3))
 (segment (start 149.7 110.22) (end 144.02 115.9) (width 0.4) (layer F.Cu) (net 3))
 (segment (start 149.7 108) (end 149.7 110.22) (width 0.4) (layer F.Cu) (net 3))
 (segment (start 117.95 98.45) (end 118 98.4) (width 0.4) (layer F.Cu) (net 4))
 (segment (start 110.1 98.45) (end 117.95 98.45) (width 0.4) (layer F.Cu) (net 4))
 (segment (start 118 103.22) (end 128.58 113.8) (width 0.4) (layer F.Cu) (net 5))
 (segment (start 118 101.375) (end 118 103.22) (width 0.4) (layer F.Cu) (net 5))
 (segment (start 163.05 104.5) (end 152.9 114.65) (width 0.4) (layer B.Cu) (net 6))
 (segment (start 152.9 114.65) (end 152.9 115.9) (width 0.4) (layer B.Cu) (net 6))
 (segment (start 169.6 104.5) (end 163.05 104.5) (width 0.4) (layer B.Cu) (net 6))
 (segment (start 171.1 103) (end 169.6 104.5) (width 0.4) (layer B.Cu) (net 6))
 (segment (start 171.4 103) (end 171.1 103) (width 0.4) (layer B.Cu) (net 6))
 (segment (start 168.5 115.84) (end 168.24 116.1) (width 0.4) (layer B.Cu) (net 7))
 (segment (start 168.5 105.975) (end 168.5 115.84) (width 0.4) (layer B.Cu) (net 7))
 (segment (start 167.7 115.56) (end 168.24 116.1) (width 0.4) (layer F.Cu) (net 7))
 (segment (start 167.7 111) (end 167.7 115.56) (width 0.4) (layer F.Cu) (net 7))
 (segment (start 173.7 113.18) (end 173.7 111) (width 0.4) (layer F.Cu) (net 8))
 (segment (start 170.78 116.1) (end 173.7 113.18) (width 0.4) (layer F.Cu) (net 8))
 (segment (start 175.7 113.72) (end 175.7 111) (width 0.4) (layer F.Cu) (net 9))
 (segment (start 173.32 116.1) (end 175.7 113.72) (width 0.4) (layer F.Cu) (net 9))
 (segment (start 115.05 103.45) (end 123.5 111.9) (width 0.4) (layer F.Cu) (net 10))
 (segment (start 123.5 111.9) (end 123.5 113.8) (width 0.4) (layer F.Cu) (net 10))
 (segment (start 110.1 103.45) (end 115.05 103.45) (width 0.4) (layer F.Cu) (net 10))
 (segment (start 160.26249 91.47501) (end 159.8125 91.925) (width 0.4) (layer F.Cu) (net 11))
 (segment (start 175.7 94.15) (end 173.02501 91.47501) (width 0.4) (layer F.Cu) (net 11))
 (segment (start 159.8125 91.925) (end 159.8125 92.8) (width 0.4) (layer F.Cu) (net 11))
 (segment (start 173.02501 91.47501) (end 160.26249 91.47501) (width 0.4) (layer F.Cu) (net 11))
 (segment (start 175.7 95.8) (end 175.7 94.15) (width 0.4) (layer F.Cu) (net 11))
 (segment (start 157.875 92.8) (end 157.85 92.825) (width 0.4) (layer F.Cu) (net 11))
 (segment (start 159.8125 92.8) (end 157.875 92.8) (width 0.4) (layer F.Cu) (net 11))
 (segment (start 172.175 95.325) (end 171.7 95.8) (width 0.4) (layer F.Cu) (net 12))
 (segment (start 171.7 94.15) (end 171.7 95.8) (width 0.4) (layer F.Cu) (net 12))
 (segment (start 170.35 92.8) (end 171.7 94.15) (width 0.4) (layer F.Cu) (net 12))
 (segment (start 167.975 92.8) (end 170.35 92.8) (width 0.4) (layer F.Cu) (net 12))
 (segment (start 171.4 106.6875) (end 169.7 108.3875) (width 0.4) (layer B.Cu) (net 13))
 (segment (start 171.4 105.975) (end 171.4 106.6875) (width 0.4) (layer B.Cu) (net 13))
 (via (at 169.7 112.8) (size 0.6) (drill 0.4) (layers F.Cu B.Cu) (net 13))
 (segment (start 169.7 108.3875) (end 169.7 112.8) (width 0.4) (layer B.Cu) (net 13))
 (segment (start 169.7 112.8) (end 169.7 111) (width 0.4) (layer F.Cu) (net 13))
 (segment (start 165.7 105.975) (end 165.7 112.8) (width 0.4) (layer B.Cu) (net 14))
 (via (at 165.7 112.8) (size 0.6) (drill 0.4) (layers F.Cu B.Cu) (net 14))
 (segment (start 165.7 111) (end 165.7 112.8) (width 0.4) (layer F.Cu) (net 14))
 (segment (start 163.7 112.65) (end 163.7 111) (width 0.4) (layer F.Cu) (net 15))
 (segment (start 162.8875 115.8) (end 163.7 114.9875) (width 0.4) (layer F.Cu) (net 15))
 (segment (start 163.7 114.9875) (end 163.7 112.65) (width 0.4) (layer F.Cu) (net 15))
 (segment (start 162.175 115.8) (end 162.8875 115.8) (width 0.4) (layer F.Cu) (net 15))
 (segment (start 169.529999 116.660003) (end 169.529999 115.270001) (width 0.4) (layer B.Cu) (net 16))
 (segment (start 168.840001 117.350001) (end 169.529999 116.660003) (width 0.4) (layer B.Cu) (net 16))
 (segment (start 151.800001 117.350001) (end 168.840001 117.350001) (width 0.4) (layer B.Cu) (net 16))
 (segment (start 150.35 115.9) (end 151.800001 117.350001) (width 0.4) (layer B.Cu) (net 16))
 (segment (start 149.1 115.9) (end 150.35 115.9) (width 0.4) (layer B.Cu) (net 16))
 (via (at 171.7 113.1) (size 0.6) (drill 0.4) (layers F.Cu B.Cu) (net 16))
 (segment (start 169.529999 115.270001) (end 171.7 113.1) (width 0.4) (layer B.Cu) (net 16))
 (segment (start 171.7 113.1) (end 171.7 111) (width 0.4) (layer F.Cu) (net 16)))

